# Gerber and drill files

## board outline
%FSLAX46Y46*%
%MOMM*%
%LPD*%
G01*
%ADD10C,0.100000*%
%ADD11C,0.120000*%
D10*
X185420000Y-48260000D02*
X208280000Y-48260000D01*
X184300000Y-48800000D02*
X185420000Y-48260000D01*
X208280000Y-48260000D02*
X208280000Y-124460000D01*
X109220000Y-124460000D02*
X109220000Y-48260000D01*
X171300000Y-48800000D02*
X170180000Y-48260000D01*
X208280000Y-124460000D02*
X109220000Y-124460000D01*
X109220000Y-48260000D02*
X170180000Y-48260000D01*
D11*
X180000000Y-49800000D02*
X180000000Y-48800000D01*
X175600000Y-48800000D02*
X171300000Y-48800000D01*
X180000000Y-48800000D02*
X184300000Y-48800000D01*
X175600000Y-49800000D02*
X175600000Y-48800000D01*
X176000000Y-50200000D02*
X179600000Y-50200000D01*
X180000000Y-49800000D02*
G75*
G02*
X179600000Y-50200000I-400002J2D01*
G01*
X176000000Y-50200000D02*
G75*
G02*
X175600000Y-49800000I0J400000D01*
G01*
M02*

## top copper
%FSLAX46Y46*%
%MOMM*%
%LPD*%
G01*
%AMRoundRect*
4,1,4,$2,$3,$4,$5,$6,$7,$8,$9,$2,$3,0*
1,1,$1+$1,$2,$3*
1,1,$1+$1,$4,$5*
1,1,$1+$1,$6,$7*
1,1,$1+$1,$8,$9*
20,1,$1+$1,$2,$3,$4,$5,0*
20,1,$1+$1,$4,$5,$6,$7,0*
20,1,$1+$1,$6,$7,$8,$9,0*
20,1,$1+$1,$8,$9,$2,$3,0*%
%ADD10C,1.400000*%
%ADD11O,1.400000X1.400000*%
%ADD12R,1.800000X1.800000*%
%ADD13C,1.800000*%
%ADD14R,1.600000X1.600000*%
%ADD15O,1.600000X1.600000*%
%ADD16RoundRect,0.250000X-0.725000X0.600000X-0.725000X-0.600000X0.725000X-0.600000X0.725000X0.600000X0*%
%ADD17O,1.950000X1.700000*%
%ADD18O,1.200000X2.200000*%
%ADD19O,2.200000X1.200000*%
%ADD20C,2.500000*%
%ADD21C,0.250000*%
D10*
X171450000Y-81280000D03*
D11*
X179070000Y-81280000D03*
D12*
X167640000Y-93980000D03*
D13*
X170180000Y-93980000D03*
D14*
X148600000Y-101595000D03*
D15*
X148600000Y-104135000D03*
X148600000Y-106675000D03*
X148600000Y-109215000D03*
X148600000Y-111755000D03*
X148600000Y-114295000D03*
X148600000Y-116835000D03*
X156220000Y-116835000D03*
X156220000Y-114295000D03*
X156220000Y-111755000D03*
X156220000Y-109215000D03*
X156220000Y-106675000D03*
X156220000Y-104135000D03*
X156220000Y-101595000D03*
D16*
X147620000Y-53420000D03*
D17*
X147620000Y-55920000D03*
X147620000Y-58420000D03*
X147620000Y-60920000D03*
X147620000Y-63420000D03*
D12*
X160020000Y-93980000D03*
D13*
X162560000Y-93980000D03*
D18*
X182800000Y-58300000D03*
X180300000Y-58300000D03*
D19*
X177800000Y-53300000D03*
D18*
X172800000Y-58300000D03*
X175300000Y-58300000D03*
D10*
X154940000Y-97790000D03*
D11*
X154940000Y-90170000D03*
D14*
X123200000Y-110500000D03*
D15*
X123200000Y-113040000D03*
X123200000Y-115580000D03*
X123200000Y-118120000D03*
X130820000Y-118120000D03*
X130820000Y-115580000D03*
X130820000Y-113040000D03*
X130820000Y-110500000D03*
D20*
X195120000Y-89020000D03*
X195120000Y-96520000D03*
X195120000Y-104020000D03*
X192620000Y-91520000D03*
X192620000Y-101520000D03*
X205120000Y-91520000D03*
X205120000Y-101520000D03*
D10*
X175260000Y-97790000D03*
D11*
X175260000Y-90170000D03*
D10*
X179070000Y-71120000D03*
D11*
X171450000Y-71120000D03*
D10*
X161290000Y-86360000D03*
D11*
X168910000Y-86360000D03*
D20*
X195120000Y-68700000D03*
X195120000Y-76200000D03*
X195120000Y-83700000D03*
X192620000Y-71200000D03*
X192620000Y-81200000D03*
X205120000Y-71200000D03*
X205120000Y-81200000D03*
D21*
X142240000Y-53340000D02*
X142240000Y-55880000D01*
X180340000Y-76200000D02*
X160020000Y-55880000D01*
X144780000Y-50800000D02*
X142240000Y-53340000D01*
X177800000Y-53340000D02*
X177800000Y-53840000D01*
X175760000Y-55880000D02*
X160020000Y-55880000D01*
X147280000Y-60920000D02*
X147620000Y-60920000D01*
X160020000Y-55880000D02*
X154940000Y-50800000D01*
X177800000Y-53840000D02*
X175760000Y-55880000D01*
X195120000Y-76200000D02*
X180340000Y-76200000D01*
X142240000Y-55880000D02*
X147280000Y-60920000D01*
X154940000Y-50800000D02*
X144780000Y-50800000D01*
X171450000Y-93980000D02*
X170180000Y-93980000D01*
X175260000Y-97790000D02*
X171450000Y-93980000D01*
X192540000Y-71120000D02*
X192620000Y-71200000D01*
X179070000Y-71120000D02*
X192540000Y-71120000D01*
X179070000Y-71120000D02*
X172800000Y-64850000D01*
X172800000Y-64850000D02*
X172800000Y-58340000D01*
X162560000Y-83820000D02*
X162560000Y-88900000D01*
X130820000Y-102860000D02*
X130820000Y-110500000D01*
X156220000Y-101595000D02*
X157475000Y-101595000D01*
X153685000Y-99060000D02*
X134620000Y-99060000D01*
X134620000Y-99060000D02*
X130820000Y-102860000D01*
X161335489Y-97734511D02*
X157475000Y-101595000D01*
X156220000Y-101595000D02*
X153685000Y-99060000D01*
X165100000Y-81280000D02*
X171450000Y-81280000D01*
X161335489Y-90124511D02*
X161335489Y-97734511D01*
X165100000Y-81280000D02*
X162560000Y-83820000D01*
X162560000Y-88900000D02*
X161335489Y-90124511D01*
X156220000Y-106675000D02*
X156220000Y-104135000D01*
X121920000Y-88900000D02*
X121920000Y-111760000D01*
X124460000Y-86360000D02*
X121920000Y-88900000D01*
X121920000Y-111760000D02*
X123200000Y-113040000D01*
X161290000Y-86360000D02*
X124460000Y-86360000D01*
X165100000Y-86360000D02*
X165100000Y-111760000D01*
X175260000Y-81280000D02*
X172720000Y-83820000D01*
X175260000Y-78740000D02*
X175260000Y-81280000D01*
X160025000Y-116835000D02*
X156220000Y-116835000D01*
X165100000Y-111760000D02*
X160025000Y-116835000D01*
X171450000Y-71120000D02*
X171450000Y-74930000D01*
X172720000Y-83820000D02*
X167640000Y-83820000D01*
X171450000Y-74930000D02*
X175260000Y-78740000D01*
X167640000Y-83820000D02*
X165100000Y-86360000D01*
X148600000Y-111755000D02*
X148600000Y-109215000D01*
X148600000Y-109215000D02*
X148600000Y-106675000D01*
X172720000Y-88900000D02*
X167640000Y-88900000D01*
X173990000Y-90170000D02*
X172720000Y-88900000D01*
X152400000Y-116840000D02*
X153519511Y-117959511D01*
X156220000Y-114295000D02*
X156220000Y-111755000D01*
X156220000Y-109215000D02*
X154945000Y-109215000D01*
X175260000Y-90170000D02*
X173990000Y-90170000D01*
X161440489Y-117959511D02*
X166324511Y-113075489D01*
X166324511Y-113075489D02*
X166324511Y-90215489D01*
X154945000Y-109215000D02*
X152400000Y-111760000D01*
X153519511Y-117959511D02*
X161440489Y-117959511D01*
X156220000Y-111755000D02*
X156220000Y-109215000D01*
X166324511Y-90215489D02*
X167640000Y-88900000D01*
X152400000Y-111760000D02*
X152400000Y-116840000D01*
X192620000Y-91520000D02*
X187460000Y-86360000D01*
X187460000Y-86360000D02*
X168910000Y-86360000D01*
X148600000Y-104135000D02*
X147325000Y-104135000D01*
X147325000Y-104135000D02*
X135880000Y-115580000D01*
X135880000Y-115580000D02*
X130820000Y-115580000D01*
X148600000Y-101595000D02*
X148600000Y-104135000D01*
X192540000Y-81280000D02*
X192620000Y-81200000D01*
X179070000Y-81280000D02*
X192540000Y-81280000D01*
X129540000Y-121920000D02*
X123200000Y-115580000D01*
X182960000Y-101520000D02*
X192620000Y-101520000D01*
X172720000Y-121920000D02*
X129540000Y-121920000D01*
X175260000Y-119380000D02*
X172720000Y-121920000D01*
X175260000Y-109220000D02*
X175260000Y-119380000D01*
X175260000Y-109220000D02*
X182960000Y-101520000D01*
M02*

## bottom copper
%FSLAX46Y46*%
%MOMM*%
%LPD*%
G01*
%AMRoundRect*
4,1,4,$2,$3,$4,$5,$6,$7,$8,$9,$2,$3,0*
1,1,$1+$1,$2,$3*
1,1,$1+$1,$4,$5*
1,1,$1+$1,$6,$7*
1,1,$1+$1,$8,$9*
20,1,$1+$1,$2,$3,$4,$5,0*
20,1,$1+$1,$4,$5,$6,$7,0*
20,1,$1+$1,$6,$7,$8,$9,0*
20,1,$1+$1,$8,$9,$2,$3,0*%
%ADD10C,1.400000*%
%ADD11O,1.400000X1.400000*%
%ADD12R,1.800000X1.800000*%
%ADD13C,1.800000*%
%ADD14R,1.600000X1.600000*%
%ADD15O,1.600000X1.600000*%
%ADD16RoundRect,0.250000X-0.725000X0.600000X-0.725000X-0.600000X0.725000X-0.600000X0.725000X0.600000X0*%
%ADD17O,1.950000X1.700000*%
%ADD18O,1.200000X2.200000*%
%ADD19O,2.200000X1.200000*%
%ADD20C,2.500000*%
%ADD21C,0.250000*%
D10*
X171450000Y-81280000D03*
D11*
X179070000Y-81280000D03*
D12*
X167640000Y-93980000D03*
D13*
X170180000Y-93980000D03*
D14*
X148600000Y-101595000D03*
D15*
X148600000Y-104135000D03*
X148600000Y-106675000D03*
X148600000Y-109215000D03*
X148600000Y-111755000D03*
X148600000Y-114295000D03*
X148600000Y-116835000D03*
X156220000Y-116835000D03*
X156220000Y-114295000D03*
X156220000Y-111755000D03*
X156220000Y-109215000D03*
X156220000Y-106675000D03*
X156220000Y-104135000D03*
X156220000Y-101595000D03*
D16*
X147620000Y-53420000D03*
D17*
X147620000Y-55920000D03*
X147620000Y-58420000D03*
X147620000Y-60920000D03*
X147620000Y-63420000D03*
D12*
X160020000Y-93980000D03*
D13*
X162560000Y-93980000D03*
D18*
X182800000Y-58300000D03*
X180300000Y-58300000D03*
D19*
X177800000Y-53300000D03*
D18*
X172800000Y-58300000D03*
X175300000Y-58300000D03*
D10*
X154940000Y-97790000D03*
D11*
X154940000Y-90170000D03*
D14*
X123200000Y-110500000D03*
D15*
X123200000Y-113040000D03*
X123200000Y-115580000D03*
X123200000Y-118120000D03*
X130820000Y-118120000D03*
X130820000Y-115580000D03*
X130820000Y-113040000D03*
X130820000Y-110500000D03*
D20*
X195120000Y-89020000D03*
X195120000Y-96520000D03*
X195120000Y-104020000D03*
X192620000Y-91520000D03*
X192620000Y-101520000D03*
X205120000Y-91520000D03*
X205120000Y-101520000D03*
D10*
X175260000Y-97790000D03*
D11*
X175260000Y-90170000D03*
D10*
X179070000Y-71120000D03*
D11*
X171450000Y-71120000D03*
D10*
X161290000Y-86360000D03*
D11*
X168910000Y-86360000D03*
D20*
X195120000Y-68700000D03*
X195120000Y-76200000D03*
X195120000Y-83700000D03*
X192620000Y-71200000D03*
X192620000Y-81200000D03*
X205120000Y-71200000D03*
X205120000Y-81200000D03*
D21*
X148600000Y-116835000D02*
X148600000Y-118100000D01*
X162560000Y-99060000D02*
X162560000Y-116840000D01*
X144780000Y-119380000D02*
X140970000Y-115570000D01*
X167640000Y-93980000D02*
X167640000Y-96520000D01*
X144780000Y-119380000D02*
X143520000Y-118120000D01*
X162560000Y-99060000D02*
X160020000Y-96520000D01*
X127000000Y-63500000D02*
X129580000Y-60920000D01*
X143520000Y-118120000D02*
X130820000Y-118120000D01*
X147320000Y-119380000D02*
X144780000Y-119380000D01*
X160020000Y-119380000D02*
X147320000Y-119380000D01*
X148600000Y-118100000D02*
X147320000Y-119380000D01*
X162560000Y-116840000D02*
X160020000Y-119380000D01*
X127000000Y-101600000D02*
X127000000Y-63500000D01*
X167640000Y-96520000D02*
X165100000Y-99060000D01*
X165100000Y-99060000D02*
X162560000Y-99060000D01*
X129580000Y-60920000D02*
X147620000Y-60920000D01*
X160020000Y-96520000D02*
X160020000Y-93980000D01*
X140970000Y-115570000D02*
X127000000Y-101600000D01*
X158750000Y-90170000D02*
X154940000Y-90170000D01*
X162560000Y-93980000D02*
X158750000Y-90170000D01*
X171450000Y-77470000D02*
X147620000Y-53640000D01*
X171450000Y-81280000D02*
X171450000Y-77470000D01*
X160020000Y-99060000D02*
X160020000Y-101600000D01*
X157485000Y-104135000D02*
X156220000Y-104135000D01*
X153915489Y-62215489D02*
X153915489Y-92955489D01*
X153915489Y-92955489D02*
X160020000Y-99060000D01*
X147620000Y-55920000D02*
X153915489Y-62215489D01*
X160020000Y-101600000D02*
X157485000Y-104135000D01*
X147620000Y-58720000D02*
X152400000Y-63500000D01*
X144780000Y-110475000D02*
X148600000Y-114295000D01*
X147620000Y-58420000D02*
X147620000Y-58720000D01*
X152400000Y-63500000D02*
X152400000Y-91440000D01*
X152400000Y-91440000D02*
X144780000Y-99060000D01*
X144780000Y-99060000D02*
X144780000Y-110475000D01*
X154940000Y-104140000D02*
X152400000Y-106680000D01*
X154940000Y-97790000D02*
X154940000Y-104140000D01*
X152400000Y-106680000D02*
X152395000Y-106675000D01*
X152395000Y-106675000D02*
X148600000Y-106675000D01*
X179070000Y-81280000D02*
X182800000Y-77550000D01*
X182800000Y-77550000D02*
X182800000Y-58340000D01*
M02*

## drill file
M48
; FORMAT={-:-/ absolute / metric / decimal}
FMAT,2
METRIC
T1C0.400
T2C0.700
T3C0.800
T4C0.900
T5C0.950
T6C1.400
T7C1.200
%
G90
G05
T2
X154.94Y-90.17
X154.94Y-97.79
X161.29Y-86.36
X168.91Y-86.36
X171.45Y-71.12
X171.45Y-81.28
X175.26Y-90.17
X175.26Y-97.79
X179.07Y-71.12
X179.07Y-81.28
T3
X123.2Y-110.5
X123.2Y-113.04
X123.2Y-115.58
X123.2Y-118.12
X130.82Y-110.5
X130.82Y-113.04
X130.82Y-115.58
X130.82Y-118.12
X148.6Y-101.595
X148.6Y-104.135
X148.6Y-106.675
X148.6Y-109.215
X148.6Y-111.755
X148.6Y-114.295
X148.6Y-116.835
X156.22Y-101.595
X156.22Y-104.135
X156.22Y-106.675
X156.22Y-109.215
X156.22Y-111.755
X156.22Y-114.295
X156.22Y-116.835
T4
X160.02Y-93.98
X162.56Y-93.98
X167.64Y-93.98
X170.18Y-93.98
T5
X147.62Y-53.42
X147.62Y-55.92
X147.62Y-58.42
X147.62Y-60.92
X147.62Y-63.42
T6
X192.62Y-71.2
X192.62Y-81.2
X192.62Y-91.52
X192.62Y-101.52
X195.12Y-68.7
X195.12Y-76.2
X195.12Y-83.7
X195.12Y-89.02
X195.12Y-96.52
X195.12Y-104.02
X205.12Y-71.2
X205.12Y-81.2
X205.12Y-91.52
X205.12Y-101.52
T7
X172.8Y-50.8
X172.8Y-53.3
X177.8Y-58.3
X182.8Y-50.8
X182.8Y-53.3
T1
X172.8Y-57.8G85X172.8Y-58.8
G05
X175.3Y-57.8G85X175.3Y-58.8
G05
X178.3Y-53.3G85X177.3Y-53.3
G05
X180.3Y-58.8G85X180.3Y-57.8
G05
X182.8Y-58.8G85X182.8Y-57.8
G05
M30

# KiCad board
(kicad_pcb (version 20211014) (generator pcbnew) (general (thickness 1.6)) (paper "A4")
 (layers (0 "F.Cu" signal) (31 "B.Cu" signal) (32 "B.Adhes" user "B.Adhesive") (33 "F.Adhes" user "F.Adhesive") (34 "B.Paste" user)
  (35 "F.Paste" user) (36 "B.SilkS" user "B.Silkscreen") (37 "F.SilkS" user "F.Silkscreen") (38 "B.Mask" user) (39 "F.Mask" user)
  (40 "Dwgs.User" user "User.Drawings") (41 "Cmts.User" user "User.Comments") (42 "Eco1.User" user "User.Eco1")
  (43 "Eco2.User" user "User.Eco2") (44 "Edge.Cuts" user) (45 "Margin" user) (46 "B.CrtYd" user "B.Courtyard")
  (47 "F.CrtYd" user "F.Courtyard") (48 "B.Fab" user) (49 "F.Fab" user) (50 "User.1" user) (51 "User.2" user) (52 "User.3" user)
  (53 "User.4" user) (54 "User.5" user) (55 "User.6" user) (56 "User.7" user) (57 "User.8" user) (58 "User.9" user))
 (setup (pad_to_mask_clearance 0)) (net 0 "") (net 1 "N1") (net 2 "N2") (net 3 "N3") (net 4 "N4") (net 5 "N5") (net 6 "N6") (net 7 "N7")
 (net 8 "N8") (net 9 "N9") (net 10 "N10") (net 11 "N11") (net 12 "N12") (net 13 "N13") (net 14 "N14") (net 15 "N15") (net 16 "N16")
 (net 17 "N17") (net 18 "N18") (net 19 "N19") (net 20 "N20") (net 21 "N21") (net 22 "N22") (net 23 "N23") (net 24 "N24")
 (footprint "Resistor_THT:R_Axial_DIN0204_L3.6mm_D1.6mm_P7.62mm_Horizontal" (layer "F.Cu") (at 171.45 81.28)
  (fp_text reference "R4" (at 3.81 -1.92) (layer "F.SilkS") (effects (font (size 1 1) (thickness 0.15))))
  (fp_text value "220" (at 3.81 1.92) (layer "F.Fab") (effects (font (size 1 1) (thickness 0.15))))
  (pad "1" thru_hole circle (at 0 0) (size 1.4 1.4) (drill 0.7) (layers *.Cu *.Mask) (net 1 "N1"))
  (pad "2" thru_hole oval (at 7.62 0) (size 1.4 1.4) (drill 0.7) (layers *.Cu *.Mask) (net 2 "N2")))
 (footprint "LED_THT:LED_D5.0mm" (layer "F.Cu") (at 167.64 93.98)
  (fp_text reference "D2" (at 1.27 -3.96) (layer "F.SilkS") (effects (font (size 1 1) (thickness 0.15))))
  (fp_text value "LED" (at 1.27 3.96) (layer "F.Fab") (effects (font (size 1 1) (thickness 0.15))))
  (pad "1" thru_hole rect (at 0 0) (size 1.8 1.8) (drill 0.9) (layers *.Cu *.Mask) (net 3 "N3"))
  (pad "2" thru_hole circle (at 2.54 0) (size 1.8 1.8) (drill 0.9) (layers *.Cu *.Mask) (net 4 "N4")))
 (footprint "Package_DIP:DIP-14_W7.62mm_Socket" (layer "F.Cu") (at 148.6 101.595)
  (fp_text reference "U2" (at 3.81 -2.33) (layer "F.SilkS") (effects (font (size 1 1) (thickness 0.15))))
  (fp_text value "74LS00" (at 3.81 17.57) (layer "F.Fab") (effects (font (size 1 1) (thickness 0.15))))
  (pad "1" thru_hole rect (at 0 0) (size 1.6 1.6) (drill 0.8) (layers *.Cu *.Mask) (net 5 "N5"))
  (pad "2" thru_hole oval (at 0 2.54) (size 1.6 1.6) (drill 0.8) (layers *.Cu *.Mask) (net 5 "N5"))
  (pad "3" thru_hole oval (at 0 5.08) (size 1.6 1.6) (drill 0.8) (layers *.Cu *.Mask) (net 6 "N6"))
  (pad "4" thru_hole oval (at 0 7.62) (size 1.6 1.6) (drill 0.8) (layers *.Cu *.Mask) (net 6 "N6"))
  (pad "5" thru_hole oval (at 0 10.16) (size 1.6 1.6) (drill 0.8) (layers *.Cu *.Mask) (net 6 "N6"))
  (pad "6" thru_hole oval (at 0 12.7) (size 1.6 1.6) (drill 0.8) (layers *.Cu *.Mask) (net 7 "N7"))
  (pad "7" thru_hole oval (at 0 15.24) (size 1.6 1.6) (drill 0.8) (layers *.Cu *.Mask) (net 3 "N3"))
  (pad "8" thru_hole oval (at 7.62 15.24) (size 1.6 1.6) (drill 0.8) (layers *.Cu *.Mask) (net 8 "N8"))
  (pad "9" thru_hole oval (at 7.62 12.7) (size 1.6 1.6) (drill 0.8) (layers *.Cu *.Mask) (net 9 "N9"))
  (pad "10" thru_hole oval (at 7.62 10.16) (size 1.6 1.6) (drill 0.8) (layers *.Cu *.Mask) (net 9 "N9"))
  (pad "11" thru_hole oval (at 7.62 7.62) (size 1.6 1.6) (drill 0.8) (layers *.Cu *.Mask) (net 9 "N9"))
  (pad "12" thru_hole oval (at 7.62 5.08) (size 1.6 1.6) (drill 0.8) (layers *.Cu *.Mask) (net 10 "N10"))
  (pad "13" thru_hole oval (at 7.62 2.54) (size 1.6 1.6) (drill 0.8) (layers *.Cu *.Mask) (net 10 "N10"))
  (pad "14" thru_hole oval (at 7.62 0) (size 1.6 1.6) (drill 0.8) (layers *.Cu *.Mask) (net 1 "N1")))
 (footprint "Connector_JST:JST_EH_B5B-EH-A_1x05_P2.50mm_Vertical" (layer "F.Cu") (at 147.62 53.42 -90)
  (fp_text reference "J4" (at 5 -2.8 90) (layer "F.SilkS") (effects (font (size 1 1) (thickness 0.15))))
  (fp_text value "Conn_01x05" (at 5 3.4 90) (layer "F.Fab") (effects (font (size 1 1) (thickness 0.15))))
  (pad "1" thru_hole roundrect (at 0 0 270) (size 1.7 1.95) (drill 0.95) (layers *.Cu *.Mask) (roundrect_rratio 0.147059) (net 1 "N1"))
  (pad "2" thru_hole oval (at 2.5 0 270) (size 1.7 1.95) (drill 0.95) (layers *.Cu *.Mask) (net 10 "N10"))
  (pad "3" thru_hole oval (at 5 0 270) (size 1.7 1.95) (drill 0.95) (layers *.Cu *.Mask) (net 7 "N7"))
  (pad "4" thru_hole oval (at 7.5 0 270) (size 1.7 1.95) (drill 0.95) (layers *.Cu *.Mask) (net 3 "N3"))
  (pad "5" thru_hole oval (at 10 0 270) (size 1.7 1.95) (drill 0.95) (layers *.Cu *.Mask) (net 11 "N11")))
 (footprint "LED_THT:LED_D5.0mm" (layer "F.Cu") (at 160.02 93.98)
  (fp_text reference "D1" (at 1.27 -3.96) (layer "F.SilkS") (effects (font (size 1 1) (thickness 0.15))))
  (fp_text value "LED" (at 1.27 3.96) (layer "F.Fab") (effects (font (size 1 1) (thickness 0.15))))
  (pad "1" thru_hole rect (at 0 0) (size 1.8 1.8) (drill 0.9) (layers *.Cu *.Mask) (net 3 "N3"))
  (pad "2" thru_hole circle (at 2.54 0) (size 1.8 1.8) (drill 0.9) (layers *.Cu *.Mask) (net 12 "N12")))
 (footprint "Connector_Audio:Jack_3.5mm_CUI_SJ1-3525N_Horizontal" (layer "F.Cu") (at 177.8 53.3 180)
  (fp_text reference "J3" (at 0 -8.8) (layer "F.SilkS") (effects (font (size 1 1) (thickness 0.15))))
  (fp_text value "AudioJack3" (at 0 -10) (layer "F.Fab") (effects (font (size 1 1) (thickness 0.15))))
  (fp_line (start -2.2 3.5) (end -2.2 4.5) (layer "Edge.Cuts") (width 0.12))
  (fp_line (start 2.2 4.5) (end 6.5 4.5) (layer "Edge.Cuts") (width 0.12))
  (fp_line (start -2.2 4.5) (end -6.5 4.5) (layer "Edge.Cuts") (width 0.12))
  (fp_line (start 2.2 3.5) (end 2.2 4.5) (layer "Edge.Cuts") (width 0.12))
  (fp_line (start 1.8 3.1) (end -1.8 3.1) (layer "Edge.Cuts") (width 0.12))
  (fp_arc (start -2.2 3.5) (mid -2.082842 3.217158) (end -1.8 3.1) (layer "Edge.Cuts") (width 0.12))
  (fp_arc (start 1.8 3.1) (mid 2.082843 3.217157) (end 2.2 3.5) (layer "Edge.Cuts") (width 0.12))
  (pad "" np_thru_hole circle (at 5 0 180) (size 1.2 1.2) (drill 1.2) (layers *.Cu))
  (pad "" np_thru_hole circle (at 0 -5 180) (size 1.2 1.2) (drill 1.2) (layers *.Cu))
  (pad "" np_thru_hole circle (at 5 2.5 180) (size 1.2 1.2) (drill 1.2) (layers *.Cu))
  (pad "" np_thru_hole circle (at -5 2.5 180) (size 1.2 1.2) (drill 1.2) (layers *.Cu))
  (pad "" np_thru_hole circle (at -5 0 180) (size 1.2 1.2) (drill 1.2) (layers *.Cu))
  (pad "R" thru_hole oval (at -5 -5 180) (size 1.2 2.2) (drill oval 0.4 1.4) (layers *.Cu *.Mask) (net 2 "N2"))
  (pad "RN" thru_hole oval (at -2.5 -5 180) (size 1.2 2.2) (drill oval 0.4 1.4) (layers *.Cu *.Mask))
  (pad "S" thru_hole oval (at 0 0 180) (size 2.2 1.2) (drill oval 1.4 0.4) (layers *.Cu *.Mask) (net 3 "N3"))
  (pad "T" thru_hole oval (at 5 -5) (size 1.2 2.2) (drill oval 0.4 1.4) (layers *.Cu *.Mask) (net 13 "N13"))
  (pad "TN" thru_hole oval (at 2.5 -5) (size 1.2 2.2) (drill oval 0.4 1.4) (layers *.Cu *.Mask)))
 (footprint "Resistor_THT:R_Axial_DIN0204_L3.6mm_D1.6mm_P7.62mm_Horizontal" (layer "F.Cu") (at 154.94 97.79 90)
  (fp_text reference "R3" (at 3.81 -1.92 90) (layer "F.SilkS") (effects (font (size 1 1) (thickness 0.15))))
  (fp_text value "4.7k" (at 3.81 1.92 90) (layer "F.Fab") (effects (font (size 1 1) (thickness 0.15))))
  (pad "1" thru_hole circle (at 0 0 90) (size 1.4 1.4) (drill 0.7) (layers *.Cu *.Mask) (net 6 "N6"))
  (pad "2" thru_hole oval (at 7.62 0 90) (size 1.4 1.4) (drill 0.7) (layers *.Cu *.Mask) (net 12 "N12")))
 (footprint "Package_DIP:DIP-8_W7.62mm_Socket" (layer "F.Cu") (at 123.2 110.5)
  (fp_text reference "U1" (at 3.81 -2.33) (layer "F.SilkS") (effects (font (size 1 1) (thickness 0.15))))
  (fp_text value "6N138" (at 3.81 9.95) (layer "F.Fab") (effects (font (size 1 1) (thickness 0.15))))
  (pad "1" thru_hole rect (at 0 0) (size 1.6 1.6) (drill 0.8) (layers *.Cu *.Mask) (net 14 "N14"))
  (pad "2" thru_hole oval (at 0 2.54) (size 1.6 1.6) (drill 0.8) (layers *.Cu *.Mask) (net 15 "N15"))
  (pad "3" thru_hole oval (at 0 5.08) (size 1.6 1.6) (drill 0.8) (layers *.Cu *.Mask) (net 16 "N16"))
  (pad "4" thru_hole oval (at 0 7.62) (size 1.6 1.6) (drill 0.8) (layers *.Cu *.Mask) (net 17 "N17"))
  (pad "5" thru_hole oval (at 7.62 7.62) (size 1.6 1.6) (drill 0.8) (layers *.Cu *.Mask) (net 3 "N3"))
  (pad "6" thru_hole oval (at 7.62 5.08) (size 1.6 1.6) (drill 0.8) (layers *.Cu *.Mask) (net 5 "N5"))
  (pad "7" thru_hole oval (at 7.62 2.54) (size 1.6 1.6) (drill 0.8) (layers *.Cu *.Mask) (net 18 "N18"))
  (pad "8" thru_hole oval (at 7.62 0) (size 1.6 1.6) (drill 0.8) (layers *.Cu *.Mask) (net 1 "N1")))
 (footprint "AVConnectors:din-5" (layer "F.Cu") (at 198.12 96.52 90)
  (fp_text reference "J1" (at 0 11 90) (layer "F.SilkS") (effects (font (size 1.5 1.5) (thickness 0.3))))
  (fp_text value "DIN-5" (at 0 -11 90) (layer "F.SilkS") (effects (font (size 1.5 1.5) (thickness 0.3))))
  (pad "1" thru_hole circle locked (at 7.5 -3 90) (size 2.5 2.5) (drill 1.4) (layers *.Cu *.Mask) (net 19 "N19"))
  (pad "2" thru_hole circle locked (at 0 -3 90) (size 2.5 2.5) (drill 1.4) (layers *.Cu *.Mask) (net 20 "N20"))
  (pad "3" thru_hole circle locked (at -7.5 -3 90) (size 2.5 2.5) (drill 1.4) (layers *.Cu *.Mask) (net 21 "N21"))
  (pad "4" thru_hole circle locked (at 5 -5.5 90) (size 2.5 2.5) (drill 1.4) (layers *.Cu *.Mask) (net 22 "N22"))
  (pad "5" thru_hole circle locked (at -5 -5.5 90) (size 2.5 2.5) (drill 1.4) (layers *.Cu *.Mask) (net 16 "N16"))
  (pad "6" thru_hole circle locked (at 5 7 90) (size 2.5 2.5) (drill 1.4) (layers *.Cu *.Mask))
  (pad "6" thru_hole circle locked (at -5 7 90) (size 2.5 2.5) (drill 1.4) (layers *.Cu *.Mask)))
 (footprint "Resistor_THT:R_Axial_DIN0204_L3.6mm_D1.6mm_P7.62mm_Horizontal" (layer "F.Cu") (at 175.26 97.79 90)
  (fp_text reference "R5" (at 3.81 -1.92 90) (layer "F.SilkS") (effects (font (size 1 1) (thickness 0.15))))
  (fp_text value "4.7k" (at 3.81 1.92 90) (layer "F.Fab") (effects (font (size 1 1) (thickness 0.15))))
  (pad "1" thru_hole circle (at 0 0 90) (size 1.4 1.4) (drill 0.7) (layers *.Cu *.Mask) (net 4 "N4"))
  (pad "2" thru_hole oval (at 7.62 0 90) (size 1.4 1.4) (drill 0.7) (layers *.Cu *.Mask) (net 9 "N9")))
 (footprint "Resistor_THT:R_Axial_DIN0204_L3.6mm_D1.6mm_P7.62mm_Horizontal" (layer "F.Cu") (at 179.07 71.12 180)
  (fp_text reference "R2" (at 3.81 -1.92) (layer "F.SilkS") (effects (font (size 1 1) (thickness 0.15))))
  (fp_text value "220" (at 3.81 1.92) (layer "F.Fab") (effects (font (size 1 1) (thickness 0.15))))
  (pad "1" thru_hole circle (at 0 0 180) (size 1.4 1.4) (drill 0.7) (layers *.Cu *.Mask) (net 13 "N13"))
  (pad "2" thru_hole oval (at 7.62 0 180) (size 1.4 1.4) (drill 0.7) (layers *.Cu *.Mask) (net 8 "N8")))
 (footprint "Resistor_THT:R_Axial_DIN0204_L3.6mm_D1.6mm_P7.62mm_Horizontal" (layer "F.Cu") (at 161.29 86.36)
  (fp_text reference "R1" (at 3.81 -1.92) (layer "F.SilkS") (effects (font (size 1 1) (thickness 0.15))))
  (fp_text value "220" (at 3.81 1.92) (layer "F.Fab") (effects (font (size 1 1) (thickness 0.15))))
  (pad "1" thru_hole circle (at 0 0) (size 1.4 1.4) (drill 0.7) (layers *.Cu *.Mask) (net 15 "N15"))
  (pad "2" thru_hole oval (at 7.62 0) (size 1.4 1.4) (drill 0.7) (layers *.Cu *.Mask) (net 22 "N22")))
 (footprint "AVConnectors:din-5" (layer "F.Cu") (at 198.12 76.2 90)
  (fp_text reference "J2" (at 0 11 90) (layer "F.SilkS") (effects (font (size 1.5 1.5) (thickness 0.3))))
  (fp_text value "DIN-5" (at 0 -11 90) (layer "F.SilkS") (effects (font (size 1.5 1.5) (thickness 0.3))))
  (pad "1" thru_hole circle locked (at 7.5 -3 90) (size 2.5 2.5) (drill 1.4) (layers *.Cu *.Mask) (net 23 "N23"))
  (pad "2" thru_hole circle locked (at 0 -3 90) (size 2.5 2.5) (drill 1.4) (layers *.Cu *.Mask) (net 3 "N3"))
  (pad "3" thru_hole circle locked (at -7.5 -3 90) (size 2.5 2.5) (drill 1.4) (layers *.Cu *.Mask) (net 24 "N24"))
  (pad "4" thru_hole circle locked (at 5 -5.5 90) (size 2.5 2.5) (drill 1.4) (layers *.Cu *.Mask) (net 13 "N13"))
  (pad "5" thru_hole circle locked (at -5 -5.5 90) (size 2.5 2.5) (drill 1.4) (layers *.Cu *.Mask) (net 2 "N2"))
  (pad "6" thru_hole circle locked (at 5 7 90) (size 2.5 2.5) (drill 1.4) (layers *.Cu *.Mask))
  (pad "6" thru_hole circle locked (at -5 7 90) (size 2.5 2.5) (drill 1.4) (layers *.Cu *.Mask)))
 (gr_line (start 185.42 48.26) (end 208.28 48.26) (layer "Edge.Cuts") (width 0.1))
 (gr_line (start 184.3 48.8) (end 185.42 48.26) (layer "Edge.Cuts") (width 0.1))
 (gr_line (start 208.28 48.26) (end 208.28 124.46) (layer "Edge.Cuts") (width 0.1))
 (gr_line (start 109.22 124.46) (end 109.22 48.26) (layer "Edge.Cuts") (width 0.1))
 (gr_line (start 171.3 48.8) (end 170.18 48.26) (layer "Edge.Cuts") (width 0.1))
 (gr_line (start 208.28 124.46) (end 109.22 124.46) (layer "Edge.Cuts") (width 0.1))
 (gr_line (start 109.22 48.26) (end 170.18 48.26) (layer "Edge.Cuts") (width 0.1))
 (segment (start 142.24 53.34) (end 142.24 55.88) (width 0.25) (layer "F.Cu") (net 3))
 (segment (start 180.34 76.2) (end 160.02 55.88) (width 0.25) (layer "F.Cu") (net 3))
 (segment (start 144.78 50.8) (end 142.24 53.34) (width 0.25) (layer "F.Cu") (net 3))
 (segment (start 177.8 53.34) (end 177.8 53.84) (width 0.25) (layer "F.Cu") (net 3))
 (segment (start 175.76 55.88) (end 160.02 55.88) (width 0.25) (layer "F.Cu") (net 3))
 (segment (start 147.28 60.92) (end 147.62 60.92) (width 0.25) (layer "F.Cu") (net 3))
 (segment (start 160.02 55.88) (end 154.94 50.8) (width 0.25) (layer "F.Cu") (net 3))
 (segment (start 177.8 53.84) (end 175.76 55.88) (width 0.25) (layer "F.Cu") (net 3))
 (segment (start 195.12 76.2) (end 180.34 76.2) (width 0.25) (layer "F.Cu") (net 3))
 (segment (start 142.24 55.88) (end 147.28 60.92) (width 0.25) (layer "F.Cu") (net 3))
 (segment (start 154.94 50.8) (end 144.78 50.8) (width 0.25) (layer "F.Cu") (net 3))
 (segment (start 148.6 116.835) (end 148.6 118.1) (width 0.25) (layer "B.Cu") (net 3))
 (segment (start 162.56 99.06) (end 162.56 116.84) (width 0.25) (layer "B.Cu") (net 3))
 (segment (start 144.78 119.38) (end 140.97 115.57) (width 0.25) (layer "B.Cu") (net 3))
 (segment (start 167.64 93.98) (end 167.64 96.52) (width 0.25) (layer "B.Cu") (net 3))
 (segment (start 144.78 119.38) (end 143.52 118.12) (width 0.25) (layer "B.Cu") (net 3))
 (segment (start 162.56 99.06) (end 160.02 96.52) (width 0.25) (layer "B.Cu") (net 3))
 (segment (start 127 63.5) (end 129.58 60.92) (width 0.25) (layer "B.Cu") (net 3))
 (segment (start 143.52 118.12) (end 130.82 118.12) (width 0.25) (layer "B.Cu") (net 3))
 (segment (start 147.32 119.38) (end 144.78 119.38) (width 0.25) (layer "B.Cu") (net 3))
 (segment (start 160.02 119.38) (end 147.32 119.38) (width 0.25) (layer "B.Cu") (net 3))
 (segment (start 148.6 118.1) (end 147.32 119.38) (width 0.25) (layer "B.Cu") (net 3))
 (segment (start 162.56 116.84) (end 160.02 119.38) (width 0.25) (layer "B.Cu") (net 3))
 (segment (start 127 101.6) (end 127 63.5) (width 0.25) (layer "B.Cu") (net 3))
 (segment (start 167.64 96.52) (end 165.1 99.06) (width 0.25) (layer "B.Cu") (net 3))
 (segment (start 165.1 99.06) (end 162.56 99.06) (width 0.25) (layer "B.Cu") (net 3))
 (segment (start 129.58 60.92) (end 147.62 60.92) (width 0.25) (layer "B.Cu") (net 3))
 (segment (start 160.02 96.52) (end 160.02 93.98) (width 0.25) (layer "B.Cu") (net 3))
 (segment (start 140.97 115.57) (end 127 101.6) (width 0.25) (layer "B.Cu") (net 3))
 (segment (start 158.75 90.17) (end 154.94 90.17) (width 0.25) (layer "B.Cu") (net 12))
 (segment (start 162.56 93.98) (end 158.75 90.17) (width 0.25) (layer "B.Cu") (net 12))
 (segment (start 171.45 93.98) (end 170.18 93.98) (width 0.25) (layer "F.Cu") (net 4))
 (segment (start 175.26 97.79) (end 171.45 93.98) (width 0.25) (layer "F.Cu") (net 4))
 (segment (start 192.54 71.12) (end 192.62 71.2) (width 0.25) (layer "F.Cu") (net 13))
 (segment (start 179.07 71.12) (end 192.54 71.12) (width 0.25) (layer "F.Cu") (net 13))
 (segment (start 179.07 71.12) (end 172.8 64.85) (width 0.25) (layer "F.Cu") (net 13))
 (segment (start 172.8 64.85) (end 172.8 58.34) (width 0.25) (layer "F.Cu") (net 13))
 (segment (start 162.56 83.82) (end 162.56 88.9) (width 0.25) (layer "F.Cu") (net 1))
 (segment (start 130.82 102.86) (end 130.82 110.5) (width 0.25) (layer "F.Cu") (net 1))
 (segment (start 156.22 101.595) (end 157.475 101.595) (width 0.25) (layer "F.Cu") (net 1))
 (segment (start 153.685 99.06) (end 134.62 99.06) (width 0.25) (layer "F.Cu") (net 1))
 (segment (start 134.62 99.06) (end 130.82 102.86) (width 0.25) (layer "F.Cu") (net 1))
 (segment (start 161.335489 97.734511) (end 157.475 101.595) (width 0.25) (layer "F.Cu") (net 1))
 (segment (start 156.22 101.595) (end 153.685 99.06) (width 0.25) (layer "F.Cu") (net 1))
 (segment (start 165.1 81.28) (end 171.45 81.28) (width 0.25) (layer "F.Cu") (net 1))
 (segment (start 161.335489 90.124511) (end 161.335489 97.734511) (width 0.25) (layer "F.Cu") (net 1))
 (segment (start 165.1 81.28) (end 162.56 83.82) (width 0.25) (layer "F.Cu") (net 1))
 (segment (start 162.56 88.9) (end 161.335489 90.124511) (width 0.25) (layer "F.Cu") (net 1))
 (segment (start 171.45 77.47) (end 147.62 53.64) (width 0.25) (layer "B.Cu") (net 1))
 (segment (start 171.45 81.28) (end 171.45 77.47) (width 0.25) (layer "B.Cu") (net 1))
 (segment (start 156.22 106.675) (end 156.22 104.135) (width 0.25) (layer "F.Cu") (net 10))
 (segment (start 160.02 99.06) (end 160.02 101.6) (width 0.25) (layer "B.Cu") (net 10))
 (segment (start 157.485 104.135) (end 156.22 104.135) (width 0.25) (layer "B.Cu") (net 10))
 (segment (start 153.915489 62.215489) (end 153.915489 92.955489) (width 0.25) (layer "B.Cu") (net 10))
 (segment (start 153.915489 92.955489) (end 160.02 99.06) (width 0.25) (layer "B.Cu") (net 10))
 (segment (start 147.62 55.92) (end 153.915489 62.215489) (width 0.25) (layer "B.Cu") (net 10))
 (segment (start 160.02 101.6) (end 157.485 104.135) (width 0.25) (layer "B.Cu") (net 10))
 (segment (start 147.62 58.72) (end 152.4 63.5) (width 0.25) (layer "B.Cu") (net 7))
 (segment (start 144.78 110.475) (end 148.6 114.295) (width 0.25) (layer "B.Cu") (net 7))
 (segment (start 147.62 58.42) (end 147.62 58.72) (width 0.25) (layer "B.Cu") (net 7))
 (segment (start 152.4 63.5) (end 152.4 91.44) (width 0.25) (layer "B.Cu") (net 7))
 (segment (start 152.4 91.44) (end 144.78 99.06) (width 0.25) (layer "B.Cu") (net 7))
 (segment (start 144.78 99.06) (end 144.78 110.475) (width 0.25) (layer "B.Cu") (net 7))
 (segment (start 121.92 88.9) (end 121.92 111.76) (width 0.25) (layer "F.Cu") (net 15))
 (segment (start 124.46 86.36) (end 121.92 88.9) (width 0.25) (layer "F.Cu") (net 15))
 (segment (start 121.92 111.76) (end 123.2 113.04) (width 0.25) (layer "F.Cu") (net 15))
 (segment (start 161.29 86.36) (end 124.46 86.36) (width 0.25) (layer "F.Cu") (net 15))
 (segment (start 165.1 86.36) (end 165.1 111.76) (width 0.25) (layer "F.Cu") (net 8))
 (segment (start 175.26 81.28) (end 172.72 83.82) (width 0.25) (layer "F.Cu") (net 8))
 (segment (start 175.26 78.74) (end 175.26 81.28) (width 0.25) (layer "F.Cu") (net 8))
 (segment (start 160.025 116.835) (end 156.22 116.835) (width 0.25) (layer "F.Cu") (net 8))
 (segment (start 165.1 111.76) (end 160.025 116.835) (width 0.25) (layer "F.Cu") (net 8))
 (segment (start 171.45 71.12) (end 171.45 74.93) (width 0.25) (layer "F.Cu") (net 8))
 (segment (start 172.72 83.82) (end 167.64 83.82) (width 0.25) (layer "F.Cu") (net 8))
 (segment (start 171.45 74.93) (end 175.26 78.74) (width 0.25) (layer "F.Cu") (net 8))
 (segment (start 167.64 83.82) (end 165.1 86.36) (width 0.25) (layer "F.Cu") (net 8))
 (segment (start 148.6 111.755) (end 148.6 109.215) (width 0.25) (layer "F.Cu") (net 6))
 (segment (start 148.6 109.215) (end 148.6 106.675) (width 0.25) (layer "F.Cu") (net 6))
 (segment (start 154.94 104.14) (end 152.4 106.68) (width 0.25) (layer "B.Cu") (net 6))
 (segment (start 154.94 97.79) (end 154.94 104.14) (width 0.25) (layer "B.Cu") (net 6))
 (segment (start 152.4 106.68) (end 152.395 106.675) (width 0.25) (layer "B.Cu") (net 6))
 (segment (start 152.395 106.675) (end 148.6 106.675) (width 0.25) (layer "B.Cu") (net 6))
 (segment (start 172.72 88.9) (end 167.64 88.9) (width 0.25) (layer "F.Cu") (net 9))
 (segment (start 173.99 90.17) (end 172.72 88.9) (width 0.25) (layer "F.Cu") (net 9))
 (segment (start 152.4 116.84) (end 153.519511 117.959511) (width 0.25) (layer "F.Cu") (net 9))
 (segment (start 156.22 114.295) (end 156.22 111.755) (width 0.25) (layer "F.Cu") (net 9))
 (segment (start 156.22 109.215) (end 154.945 109.215) (width 0.25) (layer "F.Cu") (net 9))
 (segment (start 175.26 90.17) (end 173.99 90.17) (width 0.25) (layer "F.Cu") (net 9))
 (segment (start 161.440489 117.959511) (end 166.324511 113.075489) (width 0.25) (layer "F.Cu") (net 9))
 (segment (start 166.324511 113.075489) (end 166.324511 90.215489) (width 0.25) (layer "F.Cu") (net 9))
 (segment (start 154.945 109.215) (end 152.4 111.76) (width 0.25) (layer "F.Cu") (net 9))
 (segment (start 153.519511 117.959511) (end 161.440489 117.959511) (width 0.25) (layer "F.Cu") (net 9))
 (segment (start 156.22 111.755) (end 156.22 109.215) (width 0.25) (layer "F.Cu") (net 9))
 (segment (start 166.324511 90.215489) (end 167.64 88.9) (width 0.25) (layer "F.Cu") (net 9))
 (segment (start 152.4 111.76) (end 152.4 116.84) (width 0.25) (layer "F.Cu") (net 9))
 (segment (start 192.62 91.52) (end 187.46 86.36) (width 0.25) (layer "F.Cu") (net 22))
 (segment (start 187.46 86.36) (end 168.91 86.36) (width 0.25) (layer "F.Cu") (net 22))
 (segment (start 148.6 104.135) (end 147.325 104.135) (width 0.25) (layer "F.Cu") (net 5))
 (segment (start 147.325 104.135) (end 135.88 115.58) (width 0.25) (layer "F.Cu") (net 5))
 (segment (start 135.88 115.58) (end 130.82 115.58) (width 0.25) (layer "F.Cu") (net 5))
 (segment (start 148.6 101.595) (end 148.6 104.135) (width 0.25) (layer "F.Cu") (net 5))
 (segment (start 192.54 81.28) (end 192.62 81.2) (width 0.25) (layer "F.Cu") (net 2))
 (segment (start 179.07 81.28) (end 192.54 81.28) (width 0.25) (layer "F.Cu") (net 2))
 (segment (start 179.07 81.28) (end 182.8 77.55) (width 0.25) (layer "B.Cu") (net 2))
 (segment (start 182.8 77.55) (end 182.8 58.34) (width 0.25) (layer "B.Cu") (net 2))
 (segment (start 129.54 121.92) (end 123.2 115.58) (width 0.25) (layer "F.Cu") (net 16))
 (segment (start 182.96 101.52) (end 192.62 101.52) (width 0.25) (layer "F.Cu") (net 16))
 (segment (start 172.72 121.92) (end 129.54 121.92) (width 0.25) (layer "F.Cu") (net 16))
 (segment (start 175.26 119.38) (end 172.72 121.92) (width 0.25) (layer "F.Cu") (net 16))
 (segment (start 175.26 109.22) (end 175.26 119.38) (width 0.25) (layer "F.Cu") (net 16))
 (segment (start 175.26 109.22) (end 182.96 101.52) (width 0.25) (layer "F.Cu") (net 16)))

